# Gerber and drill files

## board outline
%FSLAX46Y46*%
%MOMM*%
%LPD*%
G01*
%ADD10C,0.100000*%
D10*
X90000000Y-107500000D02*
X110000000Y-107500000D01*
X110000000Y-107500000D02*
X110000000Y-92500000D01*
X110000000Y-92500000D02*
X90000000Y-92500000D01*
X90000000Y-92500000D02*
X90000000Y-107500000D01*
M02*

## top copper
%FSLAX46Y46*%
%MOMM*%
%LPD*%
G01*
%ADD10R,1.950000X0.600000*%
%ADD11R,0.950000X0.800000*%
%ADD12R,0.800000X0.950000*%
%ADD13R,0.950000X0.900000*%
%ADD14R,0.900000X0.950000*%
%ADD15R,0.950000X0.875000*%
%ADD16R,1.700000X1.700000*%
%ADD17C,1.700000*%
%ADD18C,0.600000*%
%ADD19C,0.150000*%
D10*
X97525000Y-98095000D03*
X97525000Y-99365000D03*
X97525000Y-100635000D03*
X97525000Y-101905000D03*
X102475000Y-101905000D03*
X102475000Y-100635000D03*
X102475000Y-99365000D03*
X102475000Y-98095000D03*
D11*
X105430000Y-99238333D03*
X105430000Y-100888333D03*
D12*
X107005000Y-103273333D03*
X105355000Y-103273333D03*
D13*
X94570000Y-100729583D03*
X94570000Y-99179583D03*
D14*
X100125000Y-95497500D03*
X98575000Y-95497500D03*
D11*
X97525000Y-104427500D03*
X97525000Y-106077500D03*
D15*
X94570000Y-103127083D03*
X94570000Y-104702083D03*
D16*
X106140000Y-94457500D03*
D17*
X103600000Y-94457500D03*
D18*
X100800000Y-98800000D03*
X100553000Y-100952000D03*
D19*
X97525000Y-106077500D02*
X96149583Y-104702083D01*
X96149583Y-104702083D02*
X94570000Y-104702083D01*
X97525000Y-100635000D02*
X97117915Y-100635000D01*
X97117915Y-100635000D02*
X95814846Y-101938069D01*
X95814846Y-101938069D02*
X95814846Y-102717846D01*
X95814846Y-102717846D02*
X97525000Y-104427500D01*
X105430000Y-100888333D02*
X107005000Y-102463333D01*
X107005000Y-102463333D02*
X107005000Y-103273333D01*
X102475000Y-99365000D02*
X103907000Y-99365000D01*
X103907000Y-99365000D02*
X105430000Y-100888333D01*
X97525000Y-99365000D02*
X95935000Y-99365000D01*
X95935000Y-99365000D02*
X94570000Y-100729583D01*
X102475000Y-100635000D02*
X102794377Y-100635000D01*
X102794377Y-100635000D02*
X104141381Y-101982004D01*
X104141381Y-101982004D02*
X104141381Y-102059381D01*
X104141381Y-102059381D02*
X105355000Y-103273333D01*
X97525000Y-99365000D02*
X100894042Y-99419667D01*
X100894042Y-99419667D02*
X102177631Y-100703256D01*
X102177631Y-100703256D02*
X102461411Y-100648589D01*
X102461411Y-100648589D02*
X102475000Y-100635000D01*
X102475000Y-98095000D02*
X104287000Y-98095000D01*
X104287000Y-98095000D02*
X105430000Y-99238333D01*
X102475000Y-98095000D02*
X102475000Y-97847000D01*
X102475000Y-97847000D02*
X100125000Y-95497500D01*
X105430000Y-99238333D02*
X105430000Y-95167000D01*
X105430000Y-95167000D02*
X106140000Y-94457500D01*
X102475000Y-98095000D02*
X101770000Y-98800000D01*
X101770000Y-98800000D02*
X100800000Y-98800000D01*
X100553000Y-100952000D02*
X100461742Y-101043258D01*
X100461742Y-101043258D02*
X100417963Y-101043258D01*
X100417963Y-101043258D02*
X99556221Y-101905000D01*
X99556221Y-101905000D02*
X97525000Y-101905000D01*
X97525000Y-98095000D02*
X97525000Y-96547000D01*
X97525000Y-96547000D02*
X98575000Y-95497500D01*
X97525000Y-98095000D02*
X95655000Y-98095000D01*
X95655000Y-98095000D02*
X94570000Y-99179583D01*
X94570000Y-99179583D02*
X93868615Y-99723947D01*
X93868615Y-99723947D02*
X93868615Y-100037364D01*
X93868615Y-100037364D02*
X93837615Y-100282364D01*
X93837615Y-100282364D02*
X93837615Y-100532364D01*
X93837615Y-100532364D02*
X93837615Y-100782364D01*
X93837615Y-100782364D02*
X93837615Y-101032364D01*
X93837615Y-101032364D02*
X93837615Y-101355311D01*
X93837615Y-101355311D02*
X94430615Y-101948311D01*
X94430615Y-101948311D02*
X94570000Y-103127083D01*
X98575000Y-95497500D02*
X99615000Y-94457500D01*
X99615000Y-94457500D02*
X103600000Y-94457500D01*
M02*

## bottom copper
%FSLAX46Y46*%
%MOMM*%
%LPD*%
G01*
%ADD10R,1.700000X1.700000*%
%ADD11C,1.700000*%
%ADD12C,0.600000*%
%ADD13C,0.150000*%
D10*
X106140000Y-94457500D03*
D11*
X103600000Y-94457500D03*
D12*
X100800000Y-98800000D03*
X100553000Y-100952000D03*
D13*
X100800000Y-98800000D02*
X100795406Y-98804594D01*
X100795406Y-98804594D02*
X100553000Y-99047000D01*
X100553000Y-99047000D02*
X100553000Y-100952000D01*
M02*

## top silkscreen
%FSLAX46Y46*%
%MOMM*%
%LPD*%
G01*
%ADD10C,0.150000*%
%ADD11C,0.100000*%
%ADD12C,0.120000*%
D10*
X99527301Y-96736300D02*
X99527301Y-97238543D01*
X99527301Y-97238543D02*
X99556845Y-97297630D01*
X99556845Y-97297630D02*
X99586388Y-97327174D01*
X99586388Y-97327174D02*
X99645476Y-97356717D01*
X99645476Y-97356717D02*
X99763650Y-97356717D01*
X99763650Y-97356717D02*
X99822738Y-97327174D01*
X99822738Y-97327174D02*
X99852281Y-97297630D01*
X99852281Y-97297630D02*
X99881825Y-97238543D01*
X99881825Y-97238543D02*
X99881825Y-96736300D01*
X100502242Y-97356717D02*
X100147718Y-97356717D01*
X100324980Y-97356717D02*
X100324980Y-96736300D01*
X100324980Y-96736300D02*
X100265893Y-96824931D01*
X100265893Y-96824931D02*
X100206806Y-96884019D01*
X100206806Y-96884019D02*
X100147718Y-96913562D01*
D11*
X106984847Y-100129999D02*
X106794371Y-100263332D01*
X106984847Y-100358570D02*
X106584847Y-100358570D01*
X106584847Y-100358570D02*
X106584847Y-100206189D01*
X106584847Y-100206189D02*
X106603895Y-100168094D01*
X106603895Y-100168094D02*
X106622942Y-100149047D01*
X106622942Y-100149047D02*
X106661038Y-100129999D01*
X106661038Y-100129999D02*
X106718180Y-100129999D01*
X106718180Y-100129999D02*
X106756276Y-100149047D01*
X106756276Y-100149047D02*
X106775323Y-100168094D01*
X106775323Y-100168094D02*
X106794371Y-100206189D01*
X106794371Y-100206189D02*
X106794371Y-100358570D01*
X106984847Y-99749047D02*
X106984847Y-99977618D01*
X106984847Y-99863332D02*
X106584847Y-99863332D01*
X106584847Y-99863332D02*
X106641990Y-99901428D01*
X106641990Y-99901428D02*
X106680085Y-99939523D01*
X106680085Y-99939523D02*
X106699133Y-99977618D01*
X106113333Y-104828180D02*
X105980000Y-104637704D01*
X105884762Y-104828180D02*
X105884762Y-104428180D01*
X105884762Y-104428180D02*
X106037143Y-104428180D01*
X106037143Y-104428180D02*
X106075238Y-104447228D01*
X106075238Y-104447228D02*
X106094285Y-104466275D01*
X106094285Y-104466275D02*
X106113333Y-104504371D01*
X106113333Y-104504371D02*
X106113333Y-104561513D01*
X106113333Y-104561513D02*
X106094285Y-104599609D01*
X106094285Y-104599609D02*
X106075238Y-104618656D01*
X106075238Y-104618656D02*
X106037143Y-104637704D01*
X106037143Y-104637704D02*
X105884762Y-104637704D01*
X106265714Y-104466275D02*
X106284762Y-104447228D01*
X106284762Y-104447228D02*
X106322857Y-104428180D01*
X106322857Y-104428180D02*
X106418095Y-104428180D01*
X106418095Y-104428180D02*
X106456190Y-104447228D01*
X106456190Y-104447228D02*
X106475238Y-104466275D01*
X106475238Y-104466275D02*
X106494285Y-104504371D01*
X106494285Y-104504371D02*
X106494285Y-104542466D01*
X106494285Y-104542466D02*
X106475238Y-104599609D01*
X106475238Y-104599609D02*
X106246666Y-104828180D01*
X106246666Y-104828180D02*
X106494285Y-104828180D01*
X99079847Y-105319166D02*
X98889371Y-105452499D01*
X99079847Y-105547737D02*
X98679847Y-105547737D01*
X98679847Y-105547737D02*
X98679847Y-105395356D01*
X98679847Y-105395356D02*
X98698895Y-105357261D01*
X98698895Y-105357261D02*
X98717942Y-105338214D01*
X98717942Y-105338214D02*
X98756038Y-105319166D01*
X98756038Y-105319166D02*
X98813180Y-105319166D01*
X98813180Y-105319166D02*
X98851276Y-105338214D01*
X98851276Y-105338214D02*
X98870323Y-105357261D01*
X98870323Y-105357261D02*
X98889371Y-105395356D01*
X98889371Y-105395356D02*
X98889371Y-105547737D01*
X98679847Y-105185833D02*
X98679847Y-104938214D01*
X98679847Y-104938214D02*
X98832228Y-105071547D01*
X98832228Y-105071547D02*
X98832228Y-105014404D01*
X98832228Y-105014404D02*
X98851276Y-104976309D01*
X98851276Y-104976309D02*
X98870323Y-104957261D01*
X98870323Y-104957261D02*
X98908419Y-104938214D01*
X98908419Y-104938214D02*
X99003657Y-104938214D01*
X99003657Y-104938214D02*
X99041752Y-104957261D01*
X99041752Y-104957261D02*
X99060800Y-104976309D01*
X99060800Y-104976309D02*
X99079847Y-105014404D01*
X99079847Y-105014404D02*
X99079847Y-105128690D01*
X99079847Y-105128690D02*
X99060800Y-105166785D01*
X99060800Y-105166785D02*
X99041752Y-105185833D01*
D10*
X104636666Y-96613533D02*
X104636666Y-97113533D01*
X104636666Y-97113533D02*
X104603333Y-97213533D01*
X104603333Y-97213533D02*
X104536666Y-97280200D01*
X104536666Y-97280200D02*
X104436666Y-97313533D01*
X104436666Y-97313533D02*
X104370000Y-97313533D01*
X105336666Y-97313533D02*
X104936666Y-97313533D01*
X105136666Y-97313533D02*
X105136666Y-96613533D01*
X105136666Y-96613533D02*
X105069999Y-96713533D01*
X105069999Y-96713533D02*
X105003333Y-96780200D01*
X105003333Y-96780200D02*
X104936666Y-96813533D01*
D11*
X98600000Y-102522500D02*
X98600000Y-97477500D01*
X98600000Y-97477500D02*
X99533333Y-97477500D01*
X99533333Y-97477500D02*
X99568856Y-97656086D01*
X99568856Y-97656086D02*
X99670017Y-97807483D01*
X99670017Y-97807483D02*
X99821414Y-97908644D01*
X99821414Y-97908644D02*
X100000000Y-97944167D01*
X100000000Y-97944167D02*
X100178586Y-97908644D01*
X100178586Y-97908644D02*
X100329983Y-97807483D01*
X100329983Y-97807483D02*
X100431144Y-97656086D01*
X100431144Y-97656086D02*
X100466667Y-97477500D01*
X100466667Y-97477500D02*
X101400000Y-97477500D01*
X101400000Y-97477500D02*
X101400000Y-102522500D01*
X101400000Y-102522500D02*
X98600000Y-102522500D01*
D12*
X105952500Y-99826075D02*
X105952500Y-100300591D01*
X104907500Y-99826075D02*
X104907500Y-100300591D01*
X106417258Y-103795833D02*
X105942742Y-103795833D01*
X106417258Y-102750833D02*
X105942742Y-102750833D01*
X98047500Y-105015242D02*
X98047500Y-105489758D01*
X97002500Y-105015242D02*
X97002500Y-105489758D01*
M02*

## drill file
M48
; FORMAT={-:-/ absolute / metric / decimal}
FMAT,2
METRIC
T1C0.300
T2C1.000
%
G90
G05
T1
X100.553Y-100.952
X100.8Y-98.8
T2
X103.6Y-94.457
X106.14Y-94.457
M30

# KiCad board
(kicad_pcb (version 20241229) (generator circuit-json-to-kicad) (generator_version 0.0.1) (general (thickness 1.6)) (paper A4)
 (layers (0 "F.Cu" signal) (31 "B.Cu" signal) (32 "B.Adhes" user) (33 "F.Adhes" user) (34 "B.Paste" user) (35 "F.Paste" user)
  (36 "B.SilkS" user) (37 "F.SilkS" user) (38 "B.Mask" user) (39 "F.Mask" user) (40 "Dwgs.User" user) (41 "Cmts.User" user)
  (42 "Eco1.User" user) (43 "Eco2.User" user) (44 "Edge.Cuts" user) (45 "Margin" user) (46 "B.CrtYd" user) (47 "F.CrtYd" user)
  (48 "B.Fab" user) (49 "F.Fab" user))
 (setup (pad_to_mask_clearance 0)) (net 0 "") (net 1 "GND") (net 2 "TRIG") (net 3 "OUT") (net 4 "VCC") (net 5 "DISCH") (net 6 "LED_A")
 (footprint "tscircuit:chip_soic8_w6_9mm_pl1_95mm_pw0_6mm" (layer F.Cu) (at 100 100 0)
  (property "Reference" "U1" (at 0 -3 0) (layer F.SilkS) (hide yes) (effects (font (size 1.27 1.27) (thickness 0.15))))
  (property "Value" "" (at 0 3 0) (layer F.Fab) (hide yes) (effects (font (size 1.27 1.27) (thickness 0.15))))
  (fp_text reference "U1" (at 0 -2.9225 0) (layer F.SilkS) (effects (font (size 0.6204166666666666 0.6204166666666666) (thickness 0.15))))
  (fp_line (start -1.4000000000000001 2.5225) (end -1.4000000000000001 -2.5225) (stroke (width 0.1) (type default)) (layer F.SilkS))
  (fp_line (start -1.4000000000000001 -2.5225) (end -0.46666666666666673 -2.5225) (stroke (width 0.1) (type default)) (layer F.SilkS))
  (fp_line (start -0.46666666666666673 -2.5225) (end -0.4311437818386005 -2.3439143982296247) (stroke (width 0.1) (type default))
   (layer F.SilkS))
  (fp_line (start -0.4311437818386005 -2.3439143982296247) (end -0.3299831645537222 -2.192516835446278) (stroke (width 0.1) (type default))
   (layer F.SilkS))
  (fp_line (start -0.3299831645537222 -2.192516835446278) (end -0.17858560177037522 -2.0913562181613994) (stroke (width 0.1) (type default))
   (layer F.SilkS))
  (fp_line (start -0.17858560177037522 -2.0913562181613994) (end 2.857509198010491e-17 -2.055833333333333)
   (stroke (width 0.1) (type default)) (layer F.SilkS))
  (fp_line (start 2.857509198010491e-17 -2.055833333333333) (end 0.17858560177037527 -2.0913562181613994)
   (stroke (width 0.1) (type default)) (layer F.SilkS))
  (fp_line (start 0.17858560177037527 -2.0913562181613994) (end 0.32998316455372223 -2.192516835446278) (stroke (width 0.1) (type default))
   (layer F.SilkS))
  (fp_line (start 0.32998316455372223 -2.192516835446278) (end 0.4311437818386005 -2.3439143982296247) (stroke (width 0.1) (type default))
   (layer F.SilkS))
  (fp_line (start 0.4311437818386005 -2.3439143982296247) (end 0.46666666666666673 -2.5225) (stroke (width 0.1) (type default))
   (layer F.SilkS))
  (fp_line (start 0.46666666666666673 -2.5225) (end 1.4000000000000001 -2.5225) (stroke (width 0.1) (type default)) (layer F.SilkS))
  (fp_line (start 1.4000000000000001 -2.5225) (end 1.4000000000000001 2.5225) (stroke (width 0.1) (type default)) (layer F.SilkS))
  (fp_line (start 1.4000000000000001 2.5225) (end -1.4000000000000001 2.5225) (stroke (width 0.1) (type default)) (layer F.SilkS))
  (pad "1" smd rect (at -2.475 -1.905 0) (size 1.95 0.6) (layers F.Cu F.Mask) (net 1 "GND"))
  (pad "2" smd rect (at -2.475 -0.635 0) (size 1.95 0.6) (layers F.Cu F.Mask) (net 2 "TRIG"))
  (pad "3" smd rect (at -2.475 0.635 0) (size 1.95 0.6) (layers F.Cu F.Mask) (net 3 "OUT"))
  (pad "4" smd rect (at -2.475 1.905 0) (size 1.95 0.6) (layers F.Cu F.Mask) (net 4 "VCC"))
  (pad "5" smd rect (at 2.475 1.905 0) (size 1.95 0.6) (layers F.Cu F.Mask))
  (pad "6" smd rect (at 2.475 0.635 0) (size 1.95 0.6) (layers F.Cu F.Mask) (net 2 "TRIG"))
  (pad "7" smd rect (at 2.475 -0.635 0) (size 1.95 0.6) (layers F.Cu F.Mask) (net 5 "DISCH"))
  (pad "8" smd rect (at 2.475 -1.905 0) (size 1.95 0.6) (layers F.Cu F.Mask) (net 4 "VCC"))
  (pad "" smd rect (at -2.475 -1.905 0) (size 1.365 0.42) (layers F.Paste))
  (pad "" smd rect (at -2.475 -0.635 0) (size 1.365 0.42) (layers F.Paste))
  (pad "" smd rect (at -2.475 0.635 0) (size 1.365 0.42) (layers F.Paste))
  (pad "" smd rect (at -2.475 1.905 0) (size 1.365 0.42) (layers F.Paste))
  (pad "" smd rect (at 2.475 1.905 0) (size 1.365 0.42) (layers F.Paste))
  (pad "" smd rect (at 2.475 0.635 0) (size 1.365 0.42) (layers F.Paste))
  (pad "" smd rect (at 2.475 -0.635 0) (size 1.365 0.42) (layers F.Paste))
  (pad "" smd rect (at 2.475 -1.905 0) (size 1.365 0.42) (layers F.Paste)))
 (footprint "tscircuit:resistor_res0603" (layer F.Cu) (at 105.43 100.06333333333333 -90.00000000000001)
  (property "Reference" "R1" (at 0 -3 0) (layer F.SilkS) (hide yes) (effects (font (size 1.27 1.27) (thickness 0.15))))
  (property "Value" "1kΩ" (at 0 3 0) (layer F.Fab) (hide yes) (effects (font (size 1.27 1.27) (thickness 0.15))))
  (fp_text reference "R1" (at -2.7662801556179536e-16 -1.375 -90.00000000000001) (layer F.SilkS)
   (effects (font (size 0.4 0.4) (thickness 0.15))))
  (fp_line (start -0.2372580000000001 -0.5224999999999999) (end 0.23725799999999989 -0.5225000000000001)
   (stroke (width 0.12) (type default)) (layer F.SilkS))
  (fp_line (start -0.23725799999999989 0.5225000000000001) (end 0.2372580000000001 0.5224999999999999) (stroke (width 0.12) (type default))
   (layer F.SilkS))
  (pad "1" smd rect (at -0.825 0 0) (size 0.95 0.8) (layers F.Cu F.Mask) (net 4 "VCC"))
  (pad "2" smd rect (at 0.825 0 0) (size 0.95 0.8) (layers F.Cu F.Mask) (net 5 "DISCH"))
  (pad "" smd rect (at -0.825 0 0) (size 0.6649999999999999 0.5599999999999999) (layers F.Paste))
  (pad "" smd rect (at 0.825 0 0) (size 0.6649999999999999 0.5599999999999999) (layers F.Paste)))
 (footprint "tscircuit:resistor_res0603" (layer F.Cu) (at 106.18 103.27333333333334 180)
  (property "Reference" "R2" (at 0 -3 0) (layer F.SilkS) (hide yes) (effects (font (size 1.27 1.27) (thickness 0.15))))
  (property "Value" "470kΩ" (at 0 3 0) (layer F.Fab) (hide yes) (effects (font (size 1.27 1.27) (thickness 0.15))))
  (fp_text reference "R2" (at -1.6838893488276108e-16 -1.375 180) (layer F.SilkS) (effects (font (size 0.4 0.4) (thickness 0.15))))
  (fp_line (start -0.2372579999999998 -0.5225) (end 0.2372579999999997 -0.5225) (stroke (width 0.12) (type default)) (layer F.SilkS))
  (fp_line (start -0.2372579999999997 0.5225) (end 0.2372579999999998 0.5225) (stroke (width 0.12) (type default)) (layer F.SilkS))
  (pad "1" smd rect (at -0.8250000000000002 0 0) (size 0.8 0.95) (layers F.Cu F.Mask) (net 5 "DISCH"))
  (pad "2" smd rect (at 0.8250000000000002 -4.440892098500626e-16 0) (size 0.8 0.95) (layers F.Cu F.Mask) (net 2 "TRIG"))
  (pad "" smd rect (at -0.8250000000000002 0 0) (size 0.5599999999999999 0.6649999999999999) (layers F.Paste))
  (pad "" smd rect (at 0.8250000000000002 -4.440892098500626e-16 0) (size 0.5599999999999999 0.6649999999999999) (layers F.Paste)))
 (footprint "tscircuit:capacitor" (layer F.Cu) (at 94.57 99.95458333333333 90)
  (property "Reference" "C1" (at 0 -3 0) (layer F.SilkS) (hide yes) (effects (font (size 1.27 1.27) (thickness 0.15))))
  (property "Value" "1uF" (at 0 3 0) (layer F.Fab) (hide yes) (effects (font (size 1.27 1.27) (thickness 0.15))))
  (pad "1" smd rect (at -0.775 0 0) (size 0.95 0.9) (layers F.Cu F.Mask) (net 2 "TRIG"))
  (pad "2" smd rect (at 0.775 0 0) (size 0.95 0.9) (layers F.Cu F.Mask) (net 1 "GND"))
  (pad "" smd rect (at -0.775 0 0) (size 0.6649999999999999 0.63) (layers F.Paste))
  (pad "" smd rect (at 0.775 0 0) (size 0.6649999999999999 0.63) (layers F.Paste)))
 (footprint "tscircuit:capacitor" (layer F.Cu) (at 99.35 95.4975 180)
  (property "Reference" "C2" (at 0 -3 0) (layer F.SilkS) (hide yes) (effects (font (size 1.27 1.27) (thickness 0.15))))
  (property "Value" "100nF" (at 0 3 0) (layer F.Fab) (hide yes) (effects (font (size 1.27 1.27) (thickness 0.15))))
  (pad "1" smd rect (at -0.775 0 0) (size 0.9 0.95) (layers F.Cu F.Mask) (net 4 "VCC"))
  (pad "2" smd rect (at 0.7749999999999998 0 0) (size 0.9 0.95) (layers F.Cu F.Mask) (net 1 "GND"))
  (pad "" smd rect (at -0.775 0 0) (size 0.63 0.6649999999999999) (layers F.Paste))
  (pad "" smd rect (at 0.7749999999999998 0 0) (size 0.63 0.6649999999999999) (layers F.Paste)))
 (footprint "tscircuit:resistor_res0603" (layer F.Cu) (at 97.525 105.2525 -90.00000000000001)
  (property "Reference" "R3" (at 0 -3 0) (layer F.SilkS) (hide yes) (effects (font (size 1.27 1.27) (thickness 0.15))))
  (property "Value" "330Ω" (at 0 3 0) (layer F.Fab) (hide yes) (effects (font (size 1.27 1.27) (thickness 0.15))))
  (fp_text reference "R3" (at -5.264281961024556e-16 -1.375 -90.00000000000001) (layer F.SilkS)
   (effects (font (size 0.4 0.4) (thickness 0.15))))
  (fp_line (start -0.23725799999999994 -0.5224999999999999) (end 0.23725799999999955 -0.5225000000000001)
   (stroke (width 0.12) (type default)) (layer F.SilkS))
  (fp_line (start -0.23725799999999955 0.5225000000000001) (end 0.23725799999999994 0.5224999999999999) (stroke (width 0.12) (type default))
   (layer F.SilkS))
  (pad "1" smd rect (at -0.8250000000000002 4.440892098500626e-16 0) (size 0.95 0.8) (layers F.Cu F.Mask) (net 3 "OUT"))
  (pad "2" smd rect (at 0.8250000000000002 0 0) (size 0.95 0.8) (layers F.Cu F.Mask) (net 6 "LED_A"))
  (pad "" smd rect (at -0.8250000000000002 4.440892098500626e-16 0) (size 0.6649999999999999 0.5599999999999999) (layers F.Paste))
  (pad "" smd rect (at 0.8250000000000002 0 0) (size 0.6649999999999999 0.5599999999999999) (layers F.Paste)))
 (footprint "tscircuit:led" (layer F.Cu) (at 94.57 103.91458333333334 -90.00000000000001)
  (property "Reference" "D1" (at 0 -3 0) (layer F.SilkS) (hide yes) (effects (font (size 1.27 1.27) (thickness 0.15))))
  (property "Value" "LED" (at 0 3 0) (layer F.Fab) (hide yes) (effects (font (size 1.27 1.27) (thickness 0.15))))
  (pad "2" smd rect (at -0.7875000000000001 8.881784197001252e-16 0) (size 0.95 0.875) (layers F.Cu F.Mask) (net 1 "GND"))
  (pad "1" smd rect (at 0.7874999999999992 0 0) (size 0.95 0.875) (layers F.Cu F.Mask) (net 6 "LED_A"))
  (pad "" smd rect (at -0.7875000000000001 8.881784197001252e-16 0) (size 0.6649999999999999 0.6124999999999999) (layers F.Paste))
  (pad "" smd rect (at 0.7874999999999992 0 0) (size 0.6649999999999999 0.6124999999999999) (layers F.Paste)))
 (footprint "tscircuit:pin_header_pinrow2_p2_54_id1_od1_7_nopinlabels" (layer F.Cu) (at 104.87 94.4575 180)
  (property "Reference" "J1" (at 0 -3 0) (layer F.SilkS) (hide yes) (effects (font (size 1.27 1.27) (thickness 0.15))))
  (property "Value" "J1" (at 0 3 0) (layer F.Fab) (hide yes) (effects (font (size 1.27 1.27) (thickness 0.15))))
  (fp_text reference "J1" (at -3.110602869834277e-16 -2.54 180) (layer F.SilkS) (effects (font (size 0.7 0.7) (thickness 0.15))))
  (pad "1" thru_hole rect (at -1.2699999999999996 1.555301434917138e-16 180) (size 1.7 1.7) (drill 1) (layers *.Cu *.Mask) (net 4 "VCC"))
  (pad "2" thru_hole circle (at 1.27 -1.5553014349171386e-16 0) (size 1.7 1.7) (drill 1) (layers *.Cu *.Mask) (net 1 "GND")))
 (segment (start 97.525 106.0775) (end 96.14958333333333 104.70208333333333) (width 0.15) (layer F.Cu) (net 6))
 (segment (start 96.14958333333333 104.70208333333333) (end 94.57 104.70208333333333) (width 0.15) (layer F.Cu) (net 6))
 (segment (start 97.525 100.635) (end 97.11791492645091 100.635) (width 0.15) (layer F.Cu) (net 3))
 (segment (start 97.11791492645091 100.635) (end 95.81484617131424 101.93806875513667) (width 0.15) (layer F.Cu) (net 3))
 (segment (start 95.81484617131424 101.93806875513667) (end 95.81484617131424 102.71784617131424) (width 0.15) (layer F.Cu) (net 3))
 (segment (start 95.81484617131424 102.71784617131424) (end 97.525 104.4275) (width 0.15) (layer F.Cu) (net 3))
 (segment (start 105.43 100.88833333333334) (end 107.005 102.46333333333334) (width 0.15) (layer F.Cu) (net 5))
 (segment (start 107.005 102.46333333333334) (end 107.005 103.27333333333334) (width 0.15) (layer F.Cu) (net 5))
 (segment (start 102.475 99.365) (end 103.907 99.365) (width 0.15) (layer F.Cu) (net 5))
 (segment (start 103.907 99.365) (end 105.43 100.88833333333334) (width 0.15) (layer F.Cu) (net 5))
 (segment (start 97.525 99.365) (end 95.935 99.365) (width 0.15) (layer F.Cu) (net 2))
 (segment (start 95.935 99.365) (end 94.57 100.72958333333334) (width 0.15) (layer F.Cu) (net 2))
 (segment (start 102.475 100.635) (end 102.79437672626965 100.635) (width 0.15) (layer F.Cu) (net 2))
 (segment (start 102.79437672626965 100.635) (end 104.1413806598164 101.98200393354675) (width 0.15) (layer F.Cu) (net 2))
 (segment (start 104.1413806598164 101.98200393354675) (end 104.1413806598164 102.0593806598164) (width 0.15) (layer F.Cu) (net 2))
 (segment (start 104.1413806598164 102.0593806598164) (end 105.355 103.27333333333334) (width 0.15) (layer F.Cu) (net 2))
 (segment (start 97.525 99.365) (end 100.89404220193968 99.41966666034482) (width 0.15) (layer F.Cu) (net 2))
 (segment (start 100.89404220193968 99.41966666034482) (end 102.1776311356825 100.70325559408765) (width 0.15) (layer F.Cu) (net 2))
 (segment (start 102.1776311356825 100.70325559408765) (end 102.46141106625717 100.64858893374283) (width 0.15) (layer F.Cu) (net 2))
 (segment (start 102.46141106625717 100.64858893374283) (end 102.475 100.635) (width 0.15) (layer F.Cu) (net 2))
 (segment (start 102.475 98.095) (end 104.287 98.095) (width 0.15) (layer F.Cu) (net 4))
 (segment (start 104.287 98.095) (end 105.43 99.23833333333333) (width 0.15) (layer F.Cu) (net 4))
 (segment (start 102.475 98.095) (end 102.475 97.847) (width 0.15) (layer F.Cu) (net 4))
 (segment (start 102.475 97.847) (end 100.125 95.4975) (width 0.15) (layer F.Cu) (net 4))
 (segment (start 105.43 99.23833333333333) (end 105.43 95.167) (width 0.15) (layer F.Cu) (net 4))
 (segment (start 105.43 95.167) (end 106.14 94.4575) (width 0.15) (layer F.Cu) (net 4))
 (segment (start 102.475 98.095) (end 101.77 98.8) (width 0.15) (layer F.Cu) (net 4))
 (segment (start 101.77 98.8) (end 100.8 98.8) (width 0.15) (layer F.Cu) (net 4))
 (segment (start 100.8 98.8) (end 100.79540598919593 98.80459401080408) (width 0.15) (layer B.Cu) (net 4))
 (segment (start 100.79540598919593 98.80459401080408) (end 100.553 99.047) (width 0.15) (layer B.Cu) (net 4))
 (segment (start 100.553 99.047) (end 100.553 100.952) (width 0.15) (layer B.Cu) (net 4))
 (segment (start 100.553 100.952) (end 100.46174178252102 101.04325821747899) (width 0.15) (layer F.Cu) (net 4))
 (segment (start 100.46174178252102 101.04325821747899) (end 100.41796309174927 101.04325821747899) (width 0.15) (layer F.Cu) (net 4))
 (segment (start 100.41796309174927 101.04325821747899) (end 99.55622130922826 101.905) (width 0.15) (layer F.Cu) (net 4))
 (segment (start 99.55622130922826 101.905) (end 97.525 101.905) (width 0.15) (layer F.Cu) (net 4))
 (segment (start 97.525 98.095) (end 97.525 96.547) (width 0.15) (layer F.Cu) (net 1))
 (segment (start 97.525 96.547) (end 98.575 95.4975) (width 0.15) (layer F.Cu) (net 1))
 (segment (start 97.525 98.095) (end 95.655 98.095) (width 0.15) (layer F.Cu) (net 1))
 (segment (start 95.655 98.095) (end 94.57 99.17958333333334) (width 0.15) (layer F.Cu) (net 1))
 (segment (start 94.57 99.17958333333334) (end 93.86861505010863 99.72394687028586) (width 0.15) (layer F.Cu) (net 1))
 (segment (start 93.86861505010863 99.72394687028586) (end 93.86861505010863 100.03736353695253) (width 0.15) (layer F.Cu) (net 1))
 (segment (start 93.86861505010863 100.03736353695253) (end 93.83761505010862 100.28236353695252) (width 0.15) (layer F.Cu) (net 1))
 (segment (start 93.83761505010862 100.28236353695252) (end 93.83761505010862 100.53236353695252) (width 0.15) (layer F.Cu) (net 1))
 (segment (start 93.83761505010862 100.53236353695252) (end 93.83761505010862 100.78236353695252) (width 0.15) (layer F.Cu) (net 1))
 (segment (start 93.83761505010862 100.78236353695252) (end 93.83761505010862 101.03236353695252) (width 0.15) (layer F.Cu) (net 1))
 (segment (start 93.83761505010862 101.03236353695252) (end 93.83761505010862 101.3553107851861) (width 0.15) (layer F.Cu) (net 1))
 (segment (start 93.83761505010862 101.3553107851861) (end 94.43061505010863 101.94831078518611) (width 0.15) (layer F.Cu) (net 1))
 (segment (start 94.43061505010863 101.94831078518611) (end 94.57 103.12708333333333) (width 0.15) (layer F.Cu) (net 1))
 (segment (start 98.575 95.4975) (end 99.615 94.4575) (width 0.15) (layer F.Cu) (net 1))
 (segment (start 99.615 94.4575) (end 103.6 94.4575) (width 0.15) (layer F.Cu) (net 1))
 (gr_line (start 90 107.5) (end 110 107.5) (width 0.1) (layer Edge.Cuts))
 (gr_line (start 110 107.5) (end 110 92.5) (width 0.1) (layer Edge.Cuts))
 (gr_line (start 110 92.5) (end 90 92.5) (width 0.1) (layer Edge.Cuts))
 (gr_line (start 90 92.5) (end 90 107.5) (width 0.1) (layer Edge.Cuts))
 (via (at 100.8 98.8) (size 0.6) (drill 0.3) (layers F.Cu B.Cu) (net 4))
 (via (at 100.553 100.952) (size 0.6) (drill 0.3) (layers F.Cu B.Cu) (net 4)))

